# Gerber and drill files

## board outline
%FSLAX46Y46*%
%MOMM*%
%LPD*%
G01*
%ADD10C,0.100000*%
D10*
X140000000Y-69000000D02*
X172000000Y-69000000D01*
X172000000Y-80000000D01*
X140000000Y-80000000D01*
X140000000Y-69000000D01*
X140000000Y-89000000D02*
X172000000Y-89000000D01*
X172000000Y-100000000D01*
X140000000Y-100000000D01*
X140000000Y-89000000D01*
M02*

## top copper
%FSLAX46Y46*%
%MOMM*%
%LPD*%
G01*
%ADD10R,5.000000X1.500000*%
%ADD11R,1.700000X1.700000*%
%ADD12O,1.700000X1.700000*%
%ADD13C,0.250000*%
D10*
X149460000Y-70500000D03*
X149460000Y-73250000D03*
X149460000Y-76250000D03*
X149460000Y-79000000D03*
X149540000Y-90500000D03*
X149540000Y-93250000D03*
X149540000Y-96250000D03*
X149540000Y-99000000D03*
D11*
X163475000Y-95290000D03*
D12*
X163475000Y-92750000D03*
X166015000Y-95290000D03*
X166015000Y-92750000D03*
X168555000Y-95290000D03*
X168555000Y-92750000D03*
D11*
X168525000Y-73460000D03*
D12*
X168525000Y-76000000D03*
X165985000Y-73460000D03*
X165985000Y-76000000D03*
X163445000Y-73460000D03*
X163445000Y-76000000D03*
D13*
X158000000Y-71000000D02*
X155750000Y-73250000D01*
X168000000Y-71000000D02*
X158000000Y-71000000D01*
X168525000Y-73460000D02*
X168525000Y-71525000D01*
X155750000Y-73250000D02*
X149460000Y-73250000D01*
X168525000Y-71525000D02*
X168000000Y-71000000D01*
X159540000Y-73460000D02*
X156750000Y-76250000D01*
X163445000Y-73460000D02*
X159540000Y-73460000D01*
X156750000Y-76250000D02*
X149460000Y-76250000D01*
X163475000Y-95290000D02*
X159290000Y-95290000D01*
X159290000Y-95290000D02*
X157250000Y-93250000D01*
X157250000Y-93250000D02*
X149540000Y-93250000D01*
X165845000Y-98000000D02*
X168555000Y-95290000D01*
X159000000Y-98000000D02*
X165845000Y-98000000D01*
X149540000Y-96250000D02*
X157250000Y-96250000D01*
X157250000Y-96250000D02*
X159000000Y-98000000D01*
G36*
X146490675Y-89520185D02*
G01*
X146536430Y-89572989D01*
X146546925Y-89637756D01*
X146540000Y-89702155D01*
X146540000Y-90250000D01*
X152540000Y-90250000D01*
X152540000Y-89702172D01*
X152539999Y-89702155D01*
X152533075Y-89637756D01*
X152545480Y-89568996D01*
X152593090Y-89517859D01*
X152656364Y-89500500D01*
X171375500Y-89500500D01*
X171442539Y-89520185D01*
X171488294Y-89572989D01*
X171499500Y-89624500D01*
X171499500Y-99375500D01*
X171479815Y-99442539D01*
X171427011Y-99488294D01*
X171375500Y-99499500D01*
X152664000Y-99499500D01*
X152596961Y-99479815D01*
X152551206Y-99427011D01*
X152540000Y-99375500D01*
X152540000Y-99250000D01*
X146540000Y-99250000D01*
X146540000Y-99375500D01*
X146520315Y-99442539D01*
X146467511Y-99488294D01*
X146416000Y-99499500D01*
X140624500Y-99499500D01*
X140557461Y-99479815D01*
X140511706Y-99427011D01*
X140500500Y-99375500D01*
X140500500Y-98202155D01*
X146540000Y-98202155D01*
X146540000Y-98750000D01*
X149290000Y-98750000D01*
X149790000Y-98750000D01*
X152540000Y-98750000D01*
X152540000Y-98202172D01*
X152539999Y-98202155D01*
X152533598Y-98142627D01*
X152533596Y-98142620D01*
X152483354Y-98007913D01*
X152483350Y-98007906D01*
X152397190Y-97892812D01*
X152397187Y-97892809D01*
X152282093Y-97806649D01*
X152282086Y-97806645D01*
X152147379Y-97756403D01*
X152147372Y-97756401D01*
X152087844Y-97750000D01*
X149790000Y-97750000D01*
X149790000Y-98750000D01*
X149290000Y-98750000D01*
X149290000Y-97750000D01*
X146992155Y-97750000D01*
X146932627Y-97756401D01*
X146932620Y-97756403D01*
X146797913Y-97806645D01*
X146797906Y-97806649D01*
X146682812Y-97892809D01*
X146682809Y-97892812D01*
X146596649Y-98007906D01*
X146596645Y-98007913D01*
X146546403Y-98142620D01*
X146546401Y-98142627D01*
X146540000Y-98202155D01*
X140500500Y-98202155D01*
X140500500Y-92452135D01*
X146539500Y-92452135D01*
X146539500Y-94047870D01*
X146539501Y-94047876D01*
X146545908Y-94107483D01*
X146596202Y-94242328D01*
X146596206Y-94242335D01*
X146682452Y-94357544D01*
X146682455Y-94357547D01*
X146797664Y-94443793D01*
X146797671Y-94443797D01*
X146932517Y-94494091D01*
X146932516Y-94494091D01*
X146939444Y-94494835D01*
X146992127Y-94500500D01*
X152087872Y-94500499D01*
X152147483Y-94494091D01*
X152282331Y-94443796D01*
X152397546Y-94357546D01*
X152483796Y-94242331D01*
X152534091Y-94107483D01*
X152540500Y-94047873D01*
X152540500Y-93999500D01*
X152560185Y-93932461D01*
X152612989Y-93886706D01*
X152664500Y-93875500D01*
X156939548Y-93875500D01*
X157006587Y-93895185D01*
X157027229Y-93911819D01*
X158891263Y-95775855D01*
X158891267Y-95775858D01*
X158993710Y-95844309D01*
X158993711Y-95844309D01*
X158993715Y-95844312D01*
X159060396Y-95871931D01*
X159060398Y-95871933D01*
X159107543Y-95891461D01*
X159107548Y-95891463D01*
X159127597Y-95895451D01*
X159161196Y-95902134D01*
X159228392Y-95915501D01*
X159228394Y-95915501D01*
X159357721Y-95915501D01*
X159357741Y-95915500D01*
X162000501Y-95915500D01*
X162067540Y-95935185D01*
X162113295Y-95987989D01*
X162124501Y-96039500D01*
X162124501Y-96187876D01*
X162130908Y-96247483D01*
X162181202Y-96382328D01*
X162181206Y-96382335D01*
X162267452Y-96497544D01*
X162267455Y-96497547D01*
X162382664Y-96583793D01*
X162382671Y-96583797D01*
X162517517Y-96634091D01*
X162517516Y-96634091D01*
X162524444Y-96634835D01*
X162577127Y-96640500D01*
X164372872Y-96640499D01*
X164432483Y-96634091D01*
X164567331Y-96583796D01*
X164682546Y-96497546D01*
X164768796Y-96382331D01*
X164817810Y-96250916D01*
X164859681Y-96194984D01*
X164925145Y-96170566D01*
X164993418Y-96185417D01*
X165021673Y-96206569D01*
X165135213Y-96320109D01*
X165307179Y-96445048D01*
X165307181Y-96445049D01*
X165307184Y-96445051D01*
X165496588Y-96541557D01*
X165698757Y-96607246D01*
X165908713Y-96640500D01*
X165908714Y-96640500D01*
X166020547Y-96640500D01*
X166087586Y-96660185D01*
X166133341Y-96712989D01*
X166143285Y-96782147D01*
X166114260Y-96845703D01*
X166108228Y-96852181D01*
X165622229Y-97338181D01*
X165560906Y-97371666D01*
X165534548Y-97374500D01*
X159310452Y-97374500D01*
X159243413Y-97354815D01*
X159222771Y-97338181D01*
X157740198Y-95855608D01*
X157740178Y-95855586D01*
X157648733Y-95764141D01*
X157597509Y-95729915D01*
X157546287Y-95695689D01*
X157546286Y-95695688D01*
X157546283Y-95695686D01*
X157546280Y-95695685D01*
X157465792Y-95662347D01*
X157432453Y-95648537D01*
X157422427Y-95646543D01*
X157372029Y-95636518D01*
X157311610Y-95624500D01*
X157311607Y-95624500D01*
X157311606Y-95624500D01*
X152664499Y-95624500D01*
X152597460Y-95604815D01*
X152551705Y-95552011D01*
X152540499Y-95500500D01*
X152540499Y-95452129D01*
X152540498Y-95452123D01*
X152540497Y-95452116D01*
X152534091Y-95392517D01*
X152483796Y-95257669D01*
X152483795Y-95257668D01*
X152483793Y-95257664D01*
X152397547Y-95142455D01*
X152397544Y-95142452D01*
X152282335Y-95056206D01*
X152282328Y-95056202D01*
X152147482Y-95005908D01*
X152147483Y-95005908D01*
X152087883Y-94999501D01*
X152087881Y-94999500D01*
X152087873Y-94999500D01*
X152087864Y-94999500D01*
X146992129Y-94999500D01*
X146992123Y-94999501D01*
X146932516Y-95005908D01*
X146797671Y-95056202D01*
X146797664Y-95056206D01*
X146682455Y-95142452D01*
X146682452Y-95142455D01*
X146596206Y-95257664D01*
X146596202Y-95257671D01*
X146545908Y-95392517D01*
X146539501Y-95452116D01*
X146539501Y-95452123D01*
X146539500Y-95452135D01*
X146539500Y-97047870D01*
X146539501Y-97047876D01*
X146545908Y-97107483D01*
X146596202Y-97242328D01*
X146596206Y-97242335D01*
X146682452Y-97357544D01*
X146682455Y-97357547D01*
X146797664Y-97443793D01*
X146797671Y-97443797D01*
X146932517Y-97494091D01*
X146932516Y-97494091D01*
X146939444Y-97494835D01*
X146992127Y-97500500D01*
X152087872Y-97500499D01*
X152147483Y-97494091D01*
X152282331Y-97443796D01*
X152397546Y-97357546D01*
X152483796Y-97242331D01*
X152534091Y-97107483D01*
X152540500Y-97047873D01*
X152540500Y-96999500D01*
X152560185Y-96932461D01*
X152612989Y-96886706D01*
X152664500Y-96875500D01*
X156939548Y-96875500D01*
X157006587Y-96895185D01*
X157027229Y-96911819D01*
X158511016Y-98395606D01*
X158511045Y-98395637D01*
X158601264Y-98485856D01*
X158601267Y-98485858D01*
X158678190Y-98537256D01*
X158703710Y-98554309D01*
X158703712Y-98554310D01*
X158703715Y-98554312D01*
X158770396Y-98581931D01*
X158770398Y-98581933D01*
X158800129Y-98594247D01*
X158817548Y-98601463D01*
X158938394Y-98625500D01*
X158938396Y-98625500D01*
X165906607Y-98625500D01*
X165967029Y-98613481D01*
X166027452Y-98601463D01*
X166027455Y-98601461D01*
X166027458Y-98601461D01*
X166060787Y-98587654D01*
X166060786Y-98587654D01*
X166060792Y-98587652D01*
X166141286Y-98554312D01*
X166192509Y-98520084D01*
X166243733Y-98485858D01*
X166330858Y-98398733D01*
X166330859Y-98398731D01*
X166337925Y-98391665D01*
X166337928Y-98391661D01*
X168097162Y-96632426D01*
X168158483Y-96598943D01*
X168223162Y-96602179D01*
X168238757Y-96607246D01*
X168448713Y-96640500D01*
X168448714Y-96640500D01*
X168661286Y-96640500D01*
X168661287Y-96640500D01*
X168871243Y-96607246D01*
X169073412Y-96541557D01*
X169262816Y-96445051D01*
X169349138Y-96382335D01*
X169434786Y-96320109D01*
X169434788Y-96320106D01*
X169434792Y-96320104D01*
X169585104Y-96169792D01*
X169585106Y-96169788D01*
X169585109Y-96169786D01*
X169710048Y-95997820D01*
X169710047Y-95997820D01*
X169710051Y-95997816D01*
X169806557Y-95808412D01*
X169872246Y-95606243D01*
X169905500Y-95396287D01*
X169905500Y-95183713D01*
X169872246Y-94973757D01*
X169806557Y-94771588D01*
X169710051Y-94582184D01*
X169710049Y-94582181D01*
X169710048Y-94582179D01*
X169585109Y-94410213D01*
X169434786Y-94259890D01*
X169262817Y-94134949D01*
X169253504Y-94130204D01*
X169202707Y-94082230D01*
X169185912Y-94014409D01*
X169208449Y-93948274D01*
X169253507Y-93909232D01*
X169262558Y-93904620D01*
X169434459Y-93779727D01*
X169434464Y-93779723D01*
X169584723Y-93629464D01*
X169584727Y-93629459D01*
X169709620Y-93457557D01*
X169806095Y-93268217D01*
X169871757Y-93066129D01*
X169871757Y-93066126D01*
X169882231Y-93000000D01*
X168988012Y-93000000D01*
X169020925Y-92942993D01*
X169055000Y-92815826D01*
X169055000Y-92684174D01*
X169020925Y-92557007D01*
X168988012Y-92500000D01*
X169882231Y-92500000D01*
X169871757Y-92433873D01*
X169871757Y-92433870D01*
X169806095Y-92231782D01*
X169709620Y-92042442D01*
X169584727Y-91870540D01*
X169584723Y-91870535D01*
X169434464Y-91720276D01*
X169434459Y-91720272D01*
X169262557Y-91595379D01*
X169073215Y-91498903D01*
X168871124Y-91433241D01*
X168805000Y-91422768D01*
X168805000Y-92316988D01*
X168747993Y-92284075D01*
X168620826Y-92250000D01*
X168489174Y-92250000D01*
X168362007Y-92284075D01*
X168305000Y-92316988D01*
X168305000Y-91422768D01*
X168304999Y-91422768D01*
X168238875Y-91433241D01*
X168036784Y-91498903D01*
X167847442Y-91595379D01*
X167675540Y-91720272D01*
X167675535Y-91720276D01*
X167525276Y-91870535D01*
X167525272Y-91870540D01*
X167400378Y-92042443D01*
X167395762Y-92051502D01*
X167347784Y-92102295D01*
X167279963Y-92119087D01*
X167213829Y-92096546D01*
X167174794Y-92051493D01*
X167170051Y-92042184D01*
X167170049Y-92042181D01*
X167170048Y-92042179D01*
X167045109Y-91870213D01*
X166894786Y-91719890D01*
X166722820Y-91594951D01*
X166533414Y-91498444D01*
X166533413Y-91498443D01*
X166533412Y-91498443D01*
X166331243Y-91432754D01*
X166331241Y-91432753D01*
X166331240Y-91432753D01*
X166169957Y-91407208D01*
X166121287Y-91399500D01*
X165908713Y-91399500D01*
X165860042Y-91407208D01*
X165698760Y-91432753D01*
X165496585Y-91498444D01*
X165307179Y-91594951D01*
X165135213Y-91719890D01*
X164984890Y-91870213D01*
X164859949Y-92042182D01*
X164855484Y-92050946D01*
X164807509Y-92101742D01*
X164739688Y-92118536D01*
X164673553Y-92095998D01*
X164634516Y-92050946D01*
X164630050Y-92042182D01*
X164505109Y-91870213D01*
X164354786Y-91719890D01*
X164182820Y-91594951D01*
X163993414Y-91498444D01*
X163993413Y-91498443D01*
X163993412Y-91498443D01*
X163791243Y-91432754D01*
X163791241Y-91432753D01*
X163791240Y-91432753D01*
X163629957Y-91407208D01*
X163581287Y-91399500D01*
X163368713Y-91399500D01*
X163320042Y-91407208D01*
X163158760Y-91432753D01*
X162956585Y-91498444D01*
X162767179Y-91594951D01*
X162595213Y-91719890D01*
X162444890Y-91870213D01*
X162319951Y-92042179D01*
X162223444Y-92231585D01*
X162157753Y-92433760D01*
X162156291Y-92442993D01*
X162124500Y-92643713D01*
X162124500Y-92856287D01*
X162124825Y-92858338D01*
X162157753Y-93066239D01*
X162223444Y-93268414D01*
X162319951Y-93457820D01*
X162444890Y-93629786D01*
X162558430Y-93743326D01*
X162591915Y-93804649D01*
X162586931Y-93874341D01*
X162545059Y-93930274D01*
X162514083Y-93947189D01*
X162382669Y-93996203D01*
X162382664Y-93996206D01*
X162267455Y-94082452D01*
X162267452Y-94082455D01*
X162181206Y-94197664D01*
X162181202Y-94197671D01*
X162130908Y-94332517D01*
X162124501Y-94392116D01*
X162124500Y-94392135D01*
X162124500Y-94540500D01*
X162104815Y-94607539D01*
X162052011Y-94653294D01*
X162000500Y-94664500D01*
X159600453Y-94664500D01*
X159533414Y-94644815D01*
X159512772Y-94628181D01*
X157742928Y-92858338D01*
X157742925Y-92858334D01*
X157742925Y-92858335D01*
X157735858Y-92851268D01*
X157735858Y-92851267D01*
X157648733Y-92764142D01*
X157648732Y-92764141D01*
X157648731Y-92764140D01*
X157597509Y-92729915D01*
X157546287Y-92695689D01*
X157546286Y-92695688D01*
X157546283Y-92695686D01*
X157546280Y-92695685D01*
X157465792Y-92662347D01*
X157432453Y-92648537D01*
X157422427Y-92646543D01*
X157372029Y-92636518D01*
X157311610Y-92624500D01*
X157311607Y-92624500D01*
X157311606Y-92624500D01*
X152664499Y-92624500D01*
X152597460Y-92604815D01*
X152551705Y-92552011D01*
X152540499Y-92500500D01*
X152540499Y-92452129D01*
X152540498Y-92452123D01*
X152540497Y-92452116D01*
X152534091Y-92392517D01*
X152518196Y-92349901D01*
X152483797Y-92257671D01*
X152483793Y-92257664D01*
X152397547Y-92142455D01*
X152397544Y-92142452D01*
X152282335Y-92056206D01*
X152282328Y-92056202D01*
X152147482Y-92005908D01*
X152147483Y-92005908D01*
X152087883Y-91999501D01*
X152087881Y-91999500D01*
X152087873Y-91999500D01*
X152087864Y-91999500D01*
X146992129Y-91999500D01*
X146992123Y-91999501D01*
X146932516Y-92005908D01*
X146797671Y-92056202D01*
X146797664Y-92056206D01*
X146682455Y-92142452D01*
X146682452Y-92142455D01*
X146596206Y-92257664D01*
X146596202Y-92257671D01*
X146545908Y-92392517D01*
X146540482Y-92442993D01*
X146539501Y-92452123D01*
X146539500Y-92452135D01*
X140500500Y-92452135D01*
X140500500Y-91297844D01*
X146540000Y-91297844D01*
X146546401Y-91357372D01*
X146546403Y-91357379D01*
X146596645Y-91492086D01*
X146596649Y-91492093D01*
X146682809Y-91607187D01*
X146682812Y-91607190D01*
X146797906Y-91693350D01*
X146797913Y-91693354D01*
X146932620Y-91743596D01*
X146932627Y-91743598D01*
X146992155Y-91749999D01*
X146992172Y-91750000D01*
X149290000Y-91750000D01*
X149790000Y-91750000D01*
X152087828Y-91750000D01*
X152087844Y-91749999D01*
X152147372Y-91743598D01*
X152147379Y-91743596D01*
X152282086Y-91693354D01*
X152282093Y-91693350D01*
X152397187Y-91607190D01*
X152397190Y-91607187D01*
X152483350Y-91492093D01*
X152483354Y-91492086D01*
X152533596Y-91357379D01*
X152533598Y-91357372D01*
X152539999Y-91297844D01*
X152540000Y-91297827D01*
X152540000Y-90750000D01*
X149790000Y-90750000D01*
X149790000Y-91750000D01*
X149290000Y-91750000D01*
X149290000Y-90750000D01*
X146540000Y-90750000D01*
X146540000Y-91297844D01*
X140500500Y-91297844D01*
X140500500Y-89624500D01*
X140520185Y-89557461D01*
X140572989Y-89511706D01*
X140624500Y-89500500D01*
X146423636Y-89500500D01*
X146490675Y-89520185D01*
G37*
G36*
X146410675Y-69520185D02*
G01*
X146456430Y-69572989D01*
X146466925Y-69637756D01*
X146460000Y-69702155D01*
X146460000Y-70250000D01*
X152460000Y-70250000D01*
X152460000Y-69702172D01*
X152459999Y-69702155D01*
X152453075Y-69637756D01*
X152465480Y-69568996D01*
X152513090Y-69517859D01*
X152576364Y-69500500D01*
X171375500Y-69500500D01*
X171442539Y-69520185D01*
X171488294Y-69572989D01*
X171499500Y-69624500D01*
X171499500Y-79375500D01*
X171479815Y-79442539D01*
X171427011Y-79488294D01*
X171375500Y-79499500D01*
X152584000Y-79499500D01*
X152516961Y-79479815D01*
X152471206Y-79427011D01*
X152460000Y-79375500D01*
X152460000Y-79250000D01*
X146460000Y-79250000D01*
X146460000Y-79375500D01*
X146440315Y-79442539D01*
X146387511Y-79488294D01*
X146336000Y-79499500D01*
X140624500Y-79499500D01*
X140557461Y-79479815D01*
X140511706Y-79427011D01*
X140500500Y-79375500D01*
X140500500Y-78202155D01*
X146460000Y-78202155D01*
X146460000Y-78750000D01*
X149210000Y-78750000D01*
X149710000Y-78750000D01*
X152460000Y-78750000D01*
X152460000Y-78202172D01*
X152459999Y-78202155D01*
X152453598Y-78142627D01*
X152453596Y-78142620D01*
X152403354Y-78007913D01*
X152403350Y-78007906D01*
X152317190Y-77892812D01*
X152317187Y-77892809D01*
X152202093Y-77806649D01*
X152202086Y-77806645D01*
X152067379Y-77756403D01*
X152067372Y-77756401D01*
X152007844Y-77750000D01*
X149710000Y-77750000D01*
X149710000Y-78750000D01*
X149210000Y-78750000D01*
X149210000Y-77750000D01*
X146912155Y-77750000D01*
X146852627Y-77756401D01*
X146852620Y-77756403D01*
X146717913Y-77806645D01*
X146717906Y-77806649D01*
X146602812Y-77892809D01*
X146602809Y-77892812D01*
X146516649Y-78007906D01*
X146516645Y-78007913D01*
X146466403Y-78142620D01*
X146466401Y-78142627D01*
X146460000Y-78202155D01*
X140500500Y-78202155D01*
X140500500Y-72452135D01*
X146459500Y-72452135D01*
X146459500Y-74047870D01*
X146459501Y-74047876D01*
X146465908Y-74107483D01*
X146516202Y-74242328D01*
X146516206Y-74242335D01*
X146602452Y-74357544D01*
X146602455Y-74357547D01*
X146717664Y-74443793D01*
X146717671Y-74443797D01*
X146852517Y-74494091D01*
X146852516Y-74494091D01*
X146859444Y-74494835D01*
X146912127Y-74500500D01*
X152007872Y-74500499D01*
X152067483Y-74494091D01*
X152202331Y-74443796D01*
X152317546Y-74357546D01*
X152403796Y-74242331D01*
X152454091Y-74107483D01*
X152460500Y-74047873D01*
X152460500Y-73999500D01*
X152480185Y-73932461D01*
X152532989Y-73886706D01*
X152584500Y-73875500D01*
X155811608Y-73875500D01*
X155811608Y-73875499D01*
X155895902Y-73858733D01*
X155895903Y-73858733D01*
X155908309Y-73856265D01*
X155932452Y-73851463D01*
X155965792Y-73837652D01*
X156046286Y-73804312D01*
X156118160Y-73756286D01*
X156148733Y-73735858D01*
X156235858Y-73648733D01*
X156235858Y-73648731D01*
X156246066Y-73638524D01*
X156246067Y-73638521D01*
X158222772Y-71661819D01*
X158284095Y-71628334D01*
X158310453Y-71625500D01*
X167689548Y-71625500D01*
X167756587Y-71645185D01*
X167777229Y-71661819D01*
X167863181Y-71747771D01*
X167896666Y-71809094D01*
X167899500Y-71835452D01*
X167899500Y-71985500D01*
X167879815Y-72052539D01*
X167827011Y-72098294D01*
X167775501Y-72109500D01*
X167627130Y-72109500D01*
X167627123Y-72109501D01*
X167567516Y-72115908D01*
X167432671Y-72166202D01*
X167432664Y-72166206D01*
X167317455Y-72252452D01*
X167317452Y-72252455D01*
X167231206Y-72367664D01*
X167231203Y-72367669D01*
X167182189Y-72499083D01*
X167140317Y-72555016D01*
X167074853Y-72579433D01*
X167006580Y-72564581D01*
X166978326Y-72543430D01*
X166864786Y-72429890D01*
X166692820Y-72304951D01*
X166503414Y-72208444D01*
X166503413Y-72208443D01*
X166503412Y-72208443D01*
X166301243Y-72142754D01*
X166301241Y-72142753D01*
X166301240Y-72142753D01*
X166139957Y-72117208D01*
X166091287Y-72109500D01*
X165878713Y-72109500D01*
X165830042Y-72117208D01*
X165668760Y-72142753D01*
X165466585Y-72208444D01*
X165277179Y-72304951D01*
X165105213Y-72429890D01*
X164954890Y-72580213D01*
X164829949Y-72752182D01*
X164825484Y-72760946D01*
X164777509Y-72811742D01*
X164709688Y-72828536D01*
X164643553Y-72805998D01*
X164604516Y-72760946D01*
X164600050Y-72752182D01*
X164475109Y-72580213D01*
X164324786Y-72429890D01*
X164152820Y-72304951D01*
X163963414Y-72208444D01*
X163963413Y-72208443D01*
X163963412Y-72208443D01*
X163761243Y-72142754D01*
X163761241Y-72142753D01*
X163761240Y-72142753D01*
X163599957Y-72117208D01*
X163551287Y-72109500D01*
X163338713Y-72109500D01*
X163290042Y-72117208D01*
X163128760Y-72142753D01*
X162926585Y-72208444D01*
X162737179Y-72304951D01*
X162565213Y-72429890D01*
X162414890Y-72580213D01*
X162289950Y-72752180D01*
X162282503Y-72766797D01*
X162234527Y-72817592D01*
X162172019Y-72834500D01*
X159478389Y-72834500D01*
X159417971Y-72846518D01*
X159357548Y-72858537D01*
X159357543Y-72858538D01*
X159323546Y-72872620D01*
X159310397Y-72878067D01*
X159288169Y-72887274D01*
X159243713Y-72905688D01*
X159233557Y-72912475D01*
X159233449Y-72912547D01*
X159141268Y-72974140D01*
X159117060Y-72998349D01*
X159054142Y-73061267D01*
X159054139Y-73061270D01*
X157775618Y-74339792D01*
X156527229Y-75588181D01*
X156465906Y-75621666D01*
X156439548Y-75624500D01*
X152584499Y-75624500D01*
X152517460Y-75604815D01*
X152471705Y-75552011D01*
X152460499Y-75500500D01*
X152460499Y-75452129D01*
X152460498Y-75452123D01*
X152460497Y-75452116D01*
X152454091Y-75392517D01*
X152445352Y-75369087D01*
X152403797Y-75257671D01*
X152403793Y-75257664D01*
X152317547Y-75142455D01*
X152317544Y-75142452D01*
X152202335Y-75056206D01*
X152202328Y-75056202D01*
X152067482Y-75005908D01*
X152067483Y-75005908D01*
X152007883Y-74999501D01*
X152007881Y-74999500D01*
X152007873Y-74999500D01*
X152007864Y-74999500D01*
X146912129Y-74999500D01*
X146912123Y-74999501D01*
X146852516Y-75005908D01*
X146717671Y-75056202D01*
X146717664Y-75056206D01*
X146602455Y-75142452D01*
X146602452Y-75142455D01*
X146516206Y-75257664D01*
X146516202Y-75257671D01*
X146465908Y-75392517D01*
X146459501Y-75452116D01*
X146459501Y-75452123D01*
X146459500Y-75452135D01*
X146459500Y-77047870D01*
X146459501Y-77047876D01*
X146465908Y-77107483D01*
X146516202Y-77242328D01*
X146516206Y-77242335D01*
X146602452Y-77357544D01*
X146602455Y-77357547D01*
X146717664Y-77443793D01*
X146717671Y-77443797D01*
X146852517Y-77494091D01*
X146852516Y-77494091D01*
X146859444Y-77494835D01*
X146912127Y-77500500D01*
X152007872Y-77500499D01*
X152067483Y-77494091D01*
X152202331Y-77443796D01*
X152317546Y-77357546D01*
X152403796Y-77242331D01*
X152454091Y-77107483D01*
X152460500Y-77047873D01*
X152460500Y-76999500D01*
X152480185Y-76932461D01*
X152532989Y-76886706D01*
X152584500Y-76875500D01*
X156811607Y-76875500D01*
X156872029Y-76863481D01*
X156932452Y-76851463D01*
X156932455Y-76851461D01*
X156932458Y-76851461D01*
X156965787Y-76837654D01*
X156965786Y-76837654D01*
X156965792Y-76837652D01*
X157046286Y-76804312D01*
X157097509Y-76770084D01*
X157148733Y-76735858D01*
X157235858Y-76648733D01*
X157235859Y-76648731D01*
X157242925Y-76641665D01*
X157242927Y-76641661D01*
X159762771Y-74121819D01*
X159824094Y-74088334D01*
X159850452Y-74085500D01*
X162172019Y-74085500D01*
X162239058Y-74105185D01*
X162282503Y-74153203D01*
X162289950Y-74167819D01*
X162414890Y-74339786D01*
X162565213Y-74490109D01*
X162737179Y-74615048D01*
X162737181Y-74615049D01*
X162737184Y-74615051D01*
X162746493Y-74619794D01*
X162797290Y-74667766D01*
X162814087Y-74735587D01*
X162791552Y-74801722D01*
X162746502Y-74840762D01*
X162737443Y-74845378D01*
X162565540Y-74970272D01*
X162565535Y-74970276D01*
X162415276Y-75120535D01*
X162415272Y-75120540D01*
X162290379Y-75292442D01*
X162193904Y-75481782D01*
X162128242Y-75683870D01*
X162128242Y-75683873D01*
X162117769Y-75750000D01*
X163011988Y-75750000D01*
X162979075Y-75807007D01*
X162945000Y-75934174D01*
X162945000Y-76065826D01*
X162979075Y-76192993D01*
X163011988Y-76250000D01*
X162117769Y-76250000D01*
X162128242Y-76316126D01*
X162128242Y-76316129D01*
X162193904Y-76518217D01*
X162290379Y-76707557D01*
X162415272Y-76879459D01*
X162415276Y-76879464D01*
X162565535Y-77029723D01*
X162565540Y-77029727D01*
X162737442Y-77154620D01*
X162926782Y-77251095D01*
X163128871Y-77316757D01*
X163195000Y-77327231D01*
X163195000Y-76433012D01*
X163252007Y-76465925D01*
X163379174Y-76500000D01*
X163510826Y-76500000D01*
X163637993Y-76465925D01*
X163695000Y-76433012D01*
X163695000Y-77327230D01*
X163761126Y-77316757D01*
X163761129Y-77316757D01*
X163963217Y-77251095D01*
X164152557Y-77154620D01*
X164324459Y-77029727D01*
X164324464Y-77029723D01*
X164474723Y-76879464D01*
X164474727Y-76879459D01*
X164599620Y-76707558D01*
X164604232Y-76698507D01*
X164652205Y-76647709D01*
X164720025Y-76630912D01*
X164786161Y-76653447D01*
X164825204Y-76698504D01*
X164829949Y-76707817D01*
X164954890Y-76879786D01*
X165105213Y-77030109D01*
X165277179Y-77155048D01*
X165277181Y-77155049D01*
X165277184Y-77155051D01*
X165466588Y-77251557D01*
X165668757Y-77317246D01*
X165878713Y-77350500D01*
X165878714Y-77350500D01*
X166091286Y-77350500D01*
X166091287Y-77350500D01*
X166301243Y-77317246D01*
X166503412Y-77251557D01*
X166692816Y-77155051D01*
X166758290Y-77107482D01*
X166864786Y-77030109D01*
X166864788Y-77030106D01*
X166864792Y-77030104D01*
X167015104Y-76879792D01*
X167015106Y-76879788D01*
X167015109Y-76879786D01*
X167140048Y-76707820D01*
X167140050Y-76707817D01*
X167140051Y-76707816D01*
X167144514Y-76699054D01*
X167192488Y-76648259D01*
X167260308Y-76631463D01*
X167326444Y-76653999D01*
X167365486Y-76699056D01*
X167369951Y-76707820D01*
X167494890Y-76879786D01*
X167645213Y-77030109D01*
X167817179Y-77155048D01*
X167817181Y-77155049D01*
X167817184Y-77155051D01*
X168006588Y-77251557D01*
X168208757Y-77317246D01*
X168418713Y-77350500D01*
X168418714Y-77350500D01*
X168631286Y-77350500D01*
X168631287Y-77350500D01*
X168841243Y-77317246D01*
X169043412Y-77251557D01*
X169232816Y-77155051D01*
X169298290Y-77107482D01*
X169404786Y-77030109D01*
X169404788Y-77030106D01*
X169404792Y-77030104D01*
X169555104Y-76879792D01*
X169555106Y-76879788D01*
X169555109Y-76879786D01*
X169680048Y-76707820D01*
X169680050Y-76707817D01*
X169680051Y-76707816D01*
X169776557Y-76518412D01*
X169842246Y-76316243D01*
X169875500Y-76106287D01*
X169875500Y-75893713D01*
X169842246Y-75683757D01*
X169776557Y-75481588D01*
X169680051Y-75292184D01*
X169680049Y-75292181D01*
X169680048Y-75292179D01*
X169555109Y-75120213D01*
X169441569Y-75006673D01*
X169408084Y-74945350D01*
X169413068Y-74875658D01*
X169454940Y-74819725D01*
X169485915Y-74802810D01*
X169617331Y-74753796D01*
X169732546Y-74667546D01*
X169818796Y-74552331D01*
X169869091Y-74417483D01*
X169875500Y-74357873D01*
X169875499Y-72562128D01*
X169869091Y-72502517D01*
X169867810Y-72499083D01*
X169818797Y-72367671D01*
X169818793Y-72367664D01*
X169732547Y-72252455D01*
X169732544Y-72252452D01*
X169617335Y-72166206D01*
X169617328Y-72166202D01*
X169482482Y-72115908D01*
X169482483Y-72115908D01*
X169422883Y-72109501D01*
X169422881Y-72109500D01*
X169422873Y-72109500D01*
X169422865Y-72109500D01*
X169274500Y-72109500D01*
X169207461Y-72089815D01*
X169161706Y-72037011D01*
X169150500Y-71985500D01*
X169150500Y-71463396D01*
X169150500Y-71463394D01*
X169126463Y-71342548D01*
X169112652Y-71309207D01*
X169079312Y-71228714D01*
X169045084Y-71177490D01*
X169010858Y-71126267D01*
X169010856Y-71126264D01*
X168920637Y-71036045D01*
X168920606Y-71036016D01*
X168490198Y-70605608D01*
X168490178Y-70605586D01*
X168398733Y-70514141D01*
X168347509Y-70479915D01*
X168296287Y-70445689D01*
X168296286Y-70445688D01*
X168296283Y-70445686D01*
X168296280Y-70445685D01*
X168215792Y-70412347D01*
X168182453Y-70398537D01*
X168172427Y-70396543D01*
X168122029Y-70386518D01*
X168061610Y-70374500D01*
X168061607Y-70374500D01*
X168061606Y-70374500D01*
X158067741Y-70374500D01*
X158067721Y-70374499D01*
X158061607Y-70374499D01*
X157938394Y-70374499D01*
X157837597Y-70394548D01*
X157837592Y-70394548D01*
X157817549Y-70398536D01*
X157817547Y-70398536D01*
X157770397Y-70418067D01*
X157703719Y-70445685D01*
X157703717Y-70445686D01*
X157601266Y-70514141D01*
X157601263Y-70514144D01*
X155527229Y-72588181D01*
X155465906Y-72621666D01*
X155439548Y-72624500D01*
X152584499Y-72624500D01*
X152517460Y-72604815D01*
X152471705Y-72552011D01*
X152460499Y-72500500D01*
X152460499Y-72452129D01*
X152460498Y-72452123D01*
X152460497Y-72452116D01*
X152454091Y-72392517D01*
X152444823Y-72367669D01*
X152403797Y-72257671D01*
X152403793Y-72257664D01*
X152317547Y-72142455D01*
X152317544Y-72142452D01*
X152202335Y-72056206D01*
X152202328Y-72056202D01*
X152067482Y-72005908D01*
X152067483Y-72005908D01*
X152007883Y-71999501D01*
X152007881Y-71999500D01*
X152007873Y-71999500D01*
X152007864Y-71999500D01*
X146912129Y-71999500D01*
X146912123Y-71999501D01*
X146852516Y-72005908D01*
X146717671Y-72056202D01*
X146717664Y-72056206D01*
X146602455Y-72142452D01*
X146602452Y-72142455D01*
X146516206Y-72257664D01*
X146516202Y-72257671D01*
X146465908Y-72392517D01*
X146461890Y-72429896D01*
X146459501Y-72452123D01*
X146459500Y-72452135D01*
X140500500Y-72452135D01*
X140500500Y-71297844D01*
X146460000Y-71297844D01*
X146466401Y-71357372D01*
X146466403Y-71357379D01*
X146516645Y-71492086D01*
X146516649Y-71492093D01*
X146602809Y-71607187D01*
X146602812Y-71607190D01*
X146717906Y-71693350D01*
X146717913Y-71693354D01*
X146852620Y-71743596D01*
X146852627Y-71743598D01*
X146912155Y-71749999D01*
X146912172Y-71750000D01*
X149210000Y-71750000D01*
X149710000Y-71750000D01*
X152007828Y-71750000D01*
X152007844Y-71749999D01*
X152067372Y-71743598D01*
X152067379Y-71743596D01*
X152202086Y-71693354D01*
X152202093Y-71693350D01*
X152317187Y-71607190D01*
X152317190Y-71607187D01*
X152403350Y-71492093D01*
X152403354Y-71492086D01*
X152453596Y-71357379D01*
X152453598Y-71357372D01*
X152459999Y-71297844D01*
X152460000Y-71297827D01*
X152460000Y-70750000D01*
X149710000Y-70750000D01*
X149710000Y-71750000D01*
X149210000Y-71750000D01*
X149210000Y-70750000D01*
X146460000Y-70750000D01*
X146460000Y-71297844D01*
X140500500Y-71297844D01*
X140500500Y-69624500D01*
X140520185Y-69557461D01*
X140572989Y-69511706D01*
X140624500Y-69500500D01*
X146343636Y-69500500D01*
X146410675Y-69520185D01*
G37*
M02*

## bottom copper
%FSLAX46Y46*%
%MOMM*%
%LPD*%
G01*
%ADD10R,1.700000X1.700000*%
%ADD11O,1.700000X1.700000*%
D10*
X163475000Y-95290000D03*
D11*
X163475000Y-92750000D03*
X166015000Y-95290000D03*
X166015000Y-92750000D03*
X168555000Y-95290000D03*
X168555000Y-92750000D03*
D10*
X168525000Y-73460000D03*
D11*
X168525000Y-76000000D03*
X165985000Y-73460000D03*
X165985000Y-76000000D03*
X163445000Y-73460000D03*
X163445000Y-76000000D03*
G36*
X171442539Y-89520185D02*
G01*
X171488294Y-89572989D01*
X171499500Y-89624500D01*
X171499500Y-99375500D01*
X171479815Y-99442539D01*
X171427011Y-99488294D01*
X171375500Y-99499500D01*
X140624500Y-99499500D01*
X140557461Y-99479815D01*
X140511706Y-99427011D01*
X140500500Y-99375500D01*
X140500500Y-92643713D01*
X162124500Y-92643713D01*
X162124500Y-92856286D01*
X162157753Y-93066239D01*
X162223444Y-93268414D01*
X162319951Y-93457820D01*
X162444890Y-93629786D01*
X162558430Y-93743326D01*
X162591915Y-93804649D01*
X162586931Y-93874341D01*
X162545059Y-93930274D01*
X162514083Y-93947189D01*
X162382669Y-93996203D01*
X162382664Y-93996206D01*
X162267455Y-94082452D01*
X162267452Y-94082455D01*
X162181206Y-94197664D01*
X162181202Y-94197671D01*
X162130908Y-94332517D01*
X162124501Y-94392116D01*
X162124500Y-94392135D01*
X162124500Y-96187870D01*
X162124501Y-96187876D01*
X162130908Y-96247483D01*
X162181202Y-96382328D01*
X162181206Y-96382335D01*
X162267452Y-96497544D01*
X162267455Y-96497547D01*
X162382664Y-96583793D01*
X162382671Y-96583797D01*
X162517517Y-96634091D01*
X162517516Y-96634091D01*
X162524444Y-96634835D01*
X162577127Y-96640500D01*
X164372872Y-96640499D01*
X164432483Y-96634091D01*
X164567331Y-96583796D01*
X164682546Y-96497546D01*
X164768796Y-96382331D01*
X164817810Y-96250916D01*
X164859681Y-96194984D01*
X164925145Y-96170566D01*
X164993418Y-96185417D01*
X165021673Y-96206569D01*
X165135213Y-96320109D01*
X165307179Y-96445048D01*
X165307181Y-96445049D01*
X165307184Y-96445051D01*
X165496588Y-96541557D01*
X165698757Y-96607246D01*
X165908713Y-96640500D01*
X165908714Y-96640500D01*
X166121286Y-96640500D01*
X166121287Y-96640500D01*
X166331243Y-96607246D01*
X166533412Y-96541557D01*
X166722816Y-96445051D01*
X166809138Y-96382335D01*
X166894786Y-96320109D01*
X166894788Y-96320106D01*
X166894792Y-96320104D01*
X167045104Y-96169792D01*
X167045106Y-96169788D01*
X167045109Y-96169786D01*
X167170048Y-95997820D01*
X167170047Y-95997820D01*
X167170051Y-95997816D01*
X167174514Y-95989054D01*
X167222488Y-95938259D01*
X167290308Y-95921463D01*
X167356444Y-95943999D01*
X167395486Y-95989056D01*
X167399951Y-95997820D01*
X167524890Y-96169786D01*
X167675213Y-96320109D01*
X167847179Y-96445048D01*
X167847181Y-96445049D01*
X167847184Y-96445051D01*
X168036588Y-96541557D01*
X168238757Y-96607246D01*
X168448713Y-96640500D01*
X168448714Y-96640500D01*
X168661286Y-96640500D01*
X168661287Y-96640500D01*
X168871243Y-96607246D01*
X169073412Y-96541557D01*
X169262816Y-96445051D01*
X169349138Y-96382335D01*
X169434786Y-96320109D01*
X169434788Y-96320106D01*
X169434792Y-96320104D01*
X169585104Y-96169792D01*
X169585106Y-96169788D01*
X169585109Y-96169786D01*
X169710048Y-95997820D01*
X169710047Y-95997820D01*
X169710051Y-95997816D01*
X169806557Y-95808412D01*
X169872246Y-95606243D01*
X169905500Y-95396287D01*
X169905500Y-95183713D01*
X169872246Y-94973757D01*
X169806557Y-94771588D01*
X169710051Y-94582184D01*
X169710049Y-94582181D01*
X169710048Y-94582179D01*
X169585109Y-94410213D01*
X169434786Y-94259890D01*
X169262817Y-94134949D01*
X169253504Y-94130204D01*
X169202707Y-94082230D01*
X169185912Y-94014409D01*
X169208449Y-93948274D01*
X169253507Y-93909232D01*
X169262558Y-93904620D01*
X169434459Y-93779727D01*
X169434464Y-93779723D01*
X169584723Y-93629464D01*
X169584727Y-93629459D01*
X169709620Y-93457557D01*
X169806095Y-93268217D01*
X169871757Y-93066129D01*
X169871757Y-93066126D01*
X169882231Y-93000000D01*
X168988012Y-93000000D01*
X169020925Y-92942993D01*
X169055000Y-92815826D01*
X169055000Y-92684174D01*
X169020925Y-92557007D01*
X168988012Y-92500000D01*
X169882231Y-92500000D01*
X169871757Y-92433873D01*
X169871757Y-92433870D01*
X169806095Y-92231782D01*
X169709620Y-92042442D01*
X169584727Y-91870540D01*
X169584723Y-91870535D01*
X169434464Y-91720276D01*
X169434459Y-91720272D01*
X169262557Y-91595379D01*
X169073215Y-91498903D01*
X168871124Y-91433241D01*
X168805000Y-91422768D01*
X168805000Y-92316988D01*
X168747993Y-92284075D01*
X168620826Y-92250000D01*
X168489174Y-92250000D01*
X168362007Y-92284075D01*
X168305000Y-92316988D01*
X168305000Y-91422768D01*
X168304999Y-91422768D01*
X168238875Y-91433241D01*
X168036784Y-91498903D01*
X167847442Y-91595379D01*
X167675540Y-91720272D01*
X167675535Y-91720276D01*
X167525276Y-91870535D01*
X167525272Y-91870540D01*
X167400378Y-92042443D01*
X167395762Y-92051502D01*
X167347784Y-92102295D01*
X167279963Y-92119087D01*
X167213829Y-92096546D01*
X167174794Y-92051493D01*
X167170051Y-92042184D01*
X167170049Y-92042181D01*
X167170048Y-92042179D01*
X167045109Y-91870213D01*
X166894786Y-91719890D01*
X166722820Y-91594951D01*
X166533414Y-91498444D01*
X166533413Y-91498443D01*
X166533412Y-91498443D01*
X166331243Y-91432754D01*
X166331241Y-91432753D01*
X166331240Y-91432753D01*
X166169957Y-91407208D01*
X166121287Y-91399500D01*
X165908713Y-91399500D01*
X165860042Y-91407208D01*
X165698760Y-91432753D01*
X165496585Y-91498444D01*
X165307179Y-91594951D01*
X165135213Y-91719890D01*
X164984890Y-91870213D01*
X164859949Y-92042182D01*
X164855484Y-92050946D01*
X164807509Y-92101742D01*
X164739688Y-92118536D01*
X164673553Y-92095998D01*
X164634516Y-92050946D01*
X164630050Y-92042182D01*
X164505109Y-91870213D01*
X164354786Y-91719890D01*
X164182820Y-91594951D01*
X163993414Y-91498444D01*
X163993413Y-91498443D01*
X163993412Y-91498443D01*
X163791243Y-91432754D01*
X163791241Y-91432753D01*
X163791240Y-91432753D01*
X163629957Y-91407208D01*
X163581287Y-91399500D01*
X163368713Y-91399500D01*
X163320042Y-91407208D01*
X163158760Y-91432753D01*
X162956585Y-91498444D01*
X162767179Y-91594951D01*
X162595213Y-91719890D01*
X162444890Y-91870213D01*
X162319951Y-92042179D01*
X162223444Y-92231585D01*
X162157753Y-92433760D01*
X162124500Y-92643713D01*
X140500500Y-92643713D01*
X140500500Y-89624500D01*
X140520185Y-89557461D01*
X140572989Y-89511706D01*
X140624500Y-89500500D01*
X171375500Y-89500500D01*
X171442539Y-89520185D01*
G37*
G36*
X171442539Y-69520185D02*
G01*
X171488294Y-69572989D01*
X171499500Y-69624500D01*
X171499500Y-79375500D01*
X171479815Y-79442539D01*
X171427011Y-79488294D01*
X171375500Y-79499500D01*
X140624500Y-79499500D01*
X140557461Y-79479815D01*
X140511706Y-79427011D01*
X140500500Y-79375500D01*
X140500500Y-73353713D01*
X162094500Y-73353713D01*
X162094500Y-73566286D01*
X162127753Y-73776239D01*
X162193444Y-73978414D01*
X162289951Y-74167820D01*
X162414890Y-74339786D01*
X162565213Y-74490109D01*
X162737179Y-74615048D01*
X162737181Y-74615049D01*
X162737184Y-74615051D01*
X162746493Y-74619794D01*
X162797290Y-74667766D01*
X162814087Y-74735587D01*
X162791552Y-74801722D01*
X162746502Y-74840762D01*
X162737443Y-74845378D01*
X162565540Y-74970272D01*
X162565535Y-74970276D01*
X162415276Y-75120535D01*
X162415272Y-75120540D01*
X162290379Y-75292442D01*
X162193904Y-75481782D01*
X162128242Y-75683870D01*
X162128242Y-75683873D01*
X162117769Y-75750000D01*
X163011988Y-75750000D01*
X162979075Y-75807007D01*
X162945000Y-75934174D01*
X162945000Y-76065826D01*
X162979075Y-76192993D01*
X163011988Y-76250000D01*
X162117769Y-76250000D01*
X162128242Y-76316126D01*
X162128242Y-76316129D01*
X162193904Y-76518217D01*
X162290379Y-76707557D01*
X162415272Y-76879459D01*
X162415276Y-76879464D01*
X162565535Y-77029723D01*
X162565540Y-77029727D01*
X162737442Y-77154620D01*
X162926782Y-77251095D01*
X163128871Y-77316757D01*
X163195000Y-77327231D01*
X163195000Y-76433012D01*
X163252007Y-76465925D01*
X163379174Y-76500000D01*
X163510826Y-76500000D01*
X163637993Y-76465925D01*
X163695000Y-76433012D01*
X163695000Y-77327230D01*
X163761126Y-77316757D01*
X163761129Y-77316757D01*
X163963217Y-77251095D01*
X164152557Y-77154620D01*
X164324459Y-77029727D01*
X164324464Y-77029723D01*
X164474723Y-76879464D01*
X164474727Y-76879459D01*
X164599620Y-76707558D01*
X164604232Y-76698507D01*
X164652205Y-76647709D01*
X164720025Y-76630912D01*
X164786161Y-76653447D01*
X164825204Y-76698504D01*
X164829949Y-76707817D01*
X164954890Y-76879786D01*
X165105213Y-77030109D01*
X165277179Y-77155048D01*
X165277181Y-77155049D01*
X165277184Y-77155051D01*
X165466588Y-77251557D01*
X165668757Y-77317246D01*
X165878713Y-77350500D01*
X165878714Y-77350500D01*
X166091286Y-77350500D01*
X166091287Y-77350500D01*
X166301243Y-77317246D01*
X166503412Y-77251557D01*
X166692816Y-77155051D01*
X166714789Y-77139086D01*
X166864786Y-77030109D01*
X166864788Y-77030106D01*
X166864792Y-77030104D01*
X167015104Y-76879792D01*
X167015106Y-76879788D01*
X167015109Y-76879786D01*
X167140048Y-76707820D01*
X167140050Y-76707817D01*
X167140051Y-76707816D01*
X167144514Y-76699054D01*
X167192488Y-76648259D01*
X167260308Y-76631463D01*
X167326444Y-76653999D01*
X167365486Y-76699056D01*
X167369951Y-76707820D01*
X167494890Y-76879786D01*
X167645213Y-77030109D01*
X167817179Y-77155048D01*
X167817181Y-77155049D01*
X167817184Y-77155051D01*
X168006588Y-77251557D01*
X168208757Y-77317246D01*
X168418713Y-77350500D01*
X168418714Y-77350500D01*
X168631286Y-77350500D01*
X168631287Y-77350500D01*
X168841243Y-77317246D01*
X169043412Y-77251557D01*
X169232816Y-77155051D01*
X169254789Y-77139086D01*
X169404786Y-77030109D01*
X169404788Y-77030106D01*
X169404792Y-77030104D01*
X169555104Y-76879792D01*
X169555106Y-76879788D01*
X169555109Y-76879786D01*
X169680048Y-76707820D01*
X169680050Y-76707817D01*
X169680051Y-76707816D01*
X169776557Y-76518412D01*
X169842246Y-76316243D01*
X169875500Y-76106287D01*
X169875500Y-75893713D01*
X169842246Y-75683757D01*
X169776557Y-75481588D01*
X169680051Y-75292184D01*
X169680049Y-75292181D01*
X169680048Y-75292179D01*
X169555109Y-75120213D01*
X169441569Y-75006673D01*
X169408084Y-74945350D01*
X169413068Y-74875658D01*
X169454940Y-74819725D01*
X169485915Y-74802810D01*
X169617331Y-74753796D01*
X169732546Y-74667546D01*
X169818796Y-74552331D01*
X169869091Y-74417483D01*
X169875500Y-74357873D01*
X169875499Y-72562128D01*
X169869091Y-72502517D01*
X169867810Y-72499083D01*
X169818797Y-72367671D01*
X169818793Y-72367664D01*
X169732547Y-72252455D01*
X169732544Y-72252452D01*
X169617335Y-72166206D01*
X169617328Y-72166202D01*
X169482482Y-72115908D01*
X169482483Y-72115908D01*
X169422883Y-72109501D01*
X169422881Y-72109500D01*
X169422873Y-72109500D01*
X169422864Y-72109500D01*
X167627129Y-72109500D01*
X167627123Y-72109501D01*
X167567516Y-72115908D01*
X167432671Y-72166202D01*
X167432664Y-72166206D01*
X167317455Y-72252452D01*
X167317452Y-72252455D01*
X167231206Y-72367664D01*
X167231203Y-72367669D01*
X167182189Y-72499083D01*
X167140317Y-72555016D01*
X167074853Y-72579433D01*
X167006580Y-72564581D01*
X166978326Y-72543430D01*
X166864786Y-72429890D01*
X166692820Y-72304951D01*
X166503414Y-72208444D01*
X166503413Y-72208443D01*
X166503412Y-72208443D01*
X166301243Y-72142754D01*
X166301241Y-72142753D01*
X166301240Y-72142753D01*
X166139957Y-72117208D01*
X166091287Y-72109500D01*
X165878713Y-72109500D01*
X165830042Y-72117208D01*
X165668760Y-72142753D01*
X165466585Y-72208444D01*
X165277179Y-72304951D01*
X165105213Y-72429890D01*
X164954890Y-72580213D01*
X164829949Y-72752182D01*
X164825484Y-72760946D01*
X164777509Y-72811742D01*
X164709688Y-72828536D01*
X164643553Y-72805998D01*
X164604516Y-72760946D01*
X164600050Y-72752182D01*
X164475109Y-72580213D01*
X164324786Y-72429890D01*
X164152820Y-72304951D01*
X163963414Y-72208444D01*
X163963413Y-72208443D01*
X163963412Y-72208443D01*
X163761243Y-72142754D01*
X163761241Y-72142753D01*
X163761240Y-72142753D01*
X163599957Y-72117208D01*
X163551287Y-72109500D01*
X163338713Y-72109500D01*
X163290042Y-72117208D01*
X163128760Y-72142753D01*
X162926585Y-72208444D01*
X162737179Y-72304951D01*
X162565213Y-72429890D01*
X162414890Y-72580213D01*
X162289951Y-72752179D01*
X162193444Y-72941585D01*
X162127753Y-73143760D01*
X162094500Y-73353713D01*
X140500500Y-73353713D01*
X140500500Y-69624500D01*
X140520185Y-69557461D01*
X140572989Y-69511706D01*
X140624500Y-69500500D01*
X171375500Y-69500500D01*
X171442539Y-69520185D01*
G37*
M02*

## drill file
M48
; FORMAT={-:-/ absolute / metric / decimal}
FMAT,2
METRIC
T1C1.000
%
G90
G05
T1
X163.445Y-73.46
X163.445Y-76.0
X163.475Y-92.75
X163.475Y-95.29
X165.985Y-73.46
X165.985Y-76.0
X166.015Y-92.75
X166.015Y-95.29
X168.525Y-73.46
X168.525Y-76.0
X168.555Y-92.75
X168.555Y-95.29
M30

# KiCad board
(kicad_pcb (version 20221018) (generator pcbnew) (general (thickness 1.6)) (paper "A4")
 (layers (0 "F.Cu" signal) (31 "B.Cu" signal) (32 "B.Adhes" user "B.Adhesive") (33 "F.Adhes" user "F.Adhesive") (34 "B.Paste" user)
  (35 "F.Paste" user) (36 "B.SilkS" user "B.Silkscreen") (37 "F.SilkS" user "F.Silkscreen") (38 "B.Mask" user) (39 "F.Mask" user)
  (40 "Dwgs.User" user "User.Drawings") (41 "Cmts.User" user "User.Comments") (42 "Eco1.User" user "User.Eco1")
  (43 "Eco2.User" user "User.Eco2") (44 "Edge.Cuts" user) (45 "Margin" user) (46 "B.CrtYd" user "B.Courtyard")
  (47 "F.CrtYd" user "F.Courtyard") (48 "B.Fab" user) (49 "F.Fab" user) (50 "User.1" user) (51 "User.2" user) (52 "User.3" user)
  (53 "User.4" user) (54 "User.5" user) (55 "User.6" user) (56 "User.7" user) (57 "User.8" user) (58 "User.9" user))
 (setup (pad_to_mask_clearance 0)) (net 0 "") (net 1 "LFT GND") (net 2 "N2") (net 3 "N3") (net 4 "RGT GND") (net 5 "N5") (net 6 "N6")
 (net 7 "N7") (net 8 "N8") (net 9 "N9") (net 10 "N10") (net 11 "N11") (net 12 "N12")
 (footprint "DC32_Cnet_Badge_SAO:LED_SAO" (layer "F.Cu") (at 118.46 74.75)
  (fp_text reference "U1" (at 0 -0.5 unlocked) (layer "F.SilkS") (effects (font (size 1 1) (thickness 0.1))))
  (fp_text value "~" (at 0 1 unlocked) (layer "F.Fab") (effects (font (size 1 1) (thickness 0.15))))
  (pad "1" smd rect (at 31 -4.25) (size 5 1.5) (layers "F.Cu" "F.Paste" "F.Mask") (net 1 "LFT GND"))
  (pad "2" smd rect (at 31 -1.5) (size 5 1.5) (layers "F.Cu" "F.Paste" "F.Mask") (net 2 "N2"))
  (pad "3" smd rect (at 31 1.5) (size 5 1.5) (layers "F.Cu" "F.Paste" "F.Mask") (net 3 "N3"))
  (pad "4" smd rect (at 31 4.25) (size 5 1.5) (layers "F.Cu" "F.Paste" "F.Mask") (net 1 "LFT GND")))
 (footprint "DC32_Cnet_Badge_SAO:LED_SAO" (layer "F.Cu") (at 118.54 94.75)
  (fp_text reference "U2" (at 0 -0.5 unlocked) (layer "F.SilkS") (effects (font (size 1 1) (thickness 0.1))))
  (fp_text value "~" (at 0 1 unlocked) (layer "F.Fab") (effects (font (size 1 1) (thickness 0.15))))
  (pad "1" smd rect (at 31 -4.25) (size 5 1.5) (layers "F.Cu" "F.Paste" "F.Mask") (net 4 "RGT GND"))
  (pad "2" smd rect (at 31 -1.5) (size 5 1.5) (layers "F.Cu" "F.Paste" "F.Mask") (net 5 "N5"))
  (pad "3" smd rect (at 31 1.5) (size 5 1.5) (layers "F.Cu" "F.Paste" "F.Mask") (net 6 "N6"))
  (pad "4" smd rect (at 31 4.25) (size 5 1.5) (layers "F.Cu" "F.Paste" "F.Mask") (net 4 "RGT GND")))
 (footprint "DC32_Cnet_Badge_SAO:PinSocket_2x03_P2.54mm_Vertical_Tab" (layer "B.Cu") (at 163.475 95.29 -90)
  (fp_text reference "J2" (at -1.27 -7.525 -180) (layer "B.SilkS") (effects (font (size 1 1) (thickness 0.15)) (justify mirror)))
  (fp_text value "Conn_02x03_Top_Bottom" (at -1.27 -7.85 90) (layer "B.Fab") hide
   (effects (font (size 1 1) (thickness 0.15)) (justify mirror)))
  (pad "1" thru_hole rect (at 0 0 270) (size 1.7 1.7) (drill 1) (layers "*.Cu" "*.Mask") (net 5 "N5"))
  (pad "2" thru_hole oval (at -2.54 0 270) (size 1.7 1.7) (drill 1) (layers "*.Cu" "*.Mask") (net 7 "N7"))
  (pad "3" thru_hole oval (at 0 -2.54 270) (size 1.7 1.7) (drill 1) (layers "*.Cu" "*.Mask") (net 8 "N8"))
  (pad "4" thru_hole oval (at -2.54 -2.54 270) (size 1.7 1.7) (drill 1) (layers "*.Cu" "*.Mask") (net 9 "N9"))
  (pad "5" thru_hole oval (at 0 -5.08 270) (size 1.7 1.7) (drill 1) (layers "*.Cu" "*.Mask") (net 6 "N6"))
  (pad "6" thru_hole oval (at -2.54 -5.08 270) (size 1.7 1.7) (drill 1) (layers "*.Cu" "*.Mask") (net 4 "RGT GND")))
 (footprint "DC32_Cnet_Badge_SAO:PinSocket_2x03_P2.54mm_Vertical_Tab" (layer "B.Cu") (at 168.525 73.46 90)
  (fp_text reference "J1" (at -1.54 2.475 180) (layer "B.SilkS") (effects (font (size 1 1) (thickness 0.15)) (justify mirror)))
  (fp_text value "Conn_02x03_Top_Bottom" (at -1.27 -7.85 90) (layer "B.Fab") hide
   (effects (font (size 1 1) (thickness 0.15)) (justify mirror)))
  (pad "1" thru_hole rect (at 0 0 90) (size 1.7 1.7) (drill 1) (layers "*.Cu" "*.Mask") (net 2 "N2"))
  (pad "2" thru_hole oval (at -2.54 0 90) (size 1.7 1.7) (drill 1) (layers "*.Cu" "*.Mask") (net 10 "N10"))
  (pad "3" thru_hole oval (at 0 -2.54 90) (size 1.7 1.7) (drill 1) (layers "*.Cu" "*.Mask") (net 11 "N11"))
  (pad "4" thru_hole oval (at -2.54 -2.54 90) (size 1.7 1.7) (drill 1) (layers "*.Cu" "*.Mask") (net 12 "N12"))
  (pad "5" thru_hole oval (at 0 -5.08 90) (size 1.7 1.7) (drill 1) (layers "*.Cu" "*.Mask") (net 3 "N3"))
  (pad "6" thru_hole oval (at -2.54 -5.08 90) (size 1.7 1.7) (drill 1) (layers "*.Cu" "*.Mask") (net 1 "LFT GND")))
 (gr_rect (start 140 69) (end 172 80) (stroke (width 0.1) (type default)) (fill none) (layer "Edge.Cuts"))
 (gr_rect (start 140 89) (end 172 100) (stroke (width 0.1) (type default)) (fill none) (layer "Edge.Cuts"))
 (segment (start 158 71) (end 155.75 73.25) (width 0.25) (layer "F.Cu") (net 2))
 (segment (start 168 71) (end 158 71) (width 0.25) (layer "F.Cu") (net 2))
 (segment (start 168.525 73.46) (end 168.525 71.525) (width 0.25) (layer "F.Cu") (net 2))
 (segment (start 155.75 73.25) (end 149.46 73.25) (width 0.25) (layer "F.Cu") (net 2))
 (segment (start 168.525 71.525) (end 168 71) (width 0.25) (layer "F.Cu") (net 2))
 (segment (start 159.54 73.46) (end 156.75 76.25) (width 0.25) (layer "F.Cu") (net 3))
 (segment (start 163.445 73.46) (end 159.54 73.46) (width 0.25) (layer "F.Cu") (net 3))
 (segment (start 156.75 76.25) (end 149.46 76.25) (width 0.25) (layer "F.Cu") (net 3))
 (segment (start 163.475 95.29) (end 159.29 95.29) (width 0.25) (layer "F.Cu") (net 5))
 (segment (start 159.29 95.29) (end 157.25 93.25) (width 0.25) (layer "F.Cu") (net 5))
 (segment (start 157.25 93.25) (end 149.54 93.25) (width 0.25) (layer "F.Cu") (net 5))
 (segment (start 165.845 98) (end 168.555 95.29) (width 0.25) (layer "F.Cu") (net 6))
 (segment (start 159 98) (end 165.845 98) (width 0.25) (layer "F.Cu") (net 6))
 (segment (start 149.54 96.25) (end 157.25 96.25) (width 0.25) (layer "F.Cu") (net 6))
 (segment (start 157.25 96.25) (end 159 98) (width 0.25) (layer "F.Cu") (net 6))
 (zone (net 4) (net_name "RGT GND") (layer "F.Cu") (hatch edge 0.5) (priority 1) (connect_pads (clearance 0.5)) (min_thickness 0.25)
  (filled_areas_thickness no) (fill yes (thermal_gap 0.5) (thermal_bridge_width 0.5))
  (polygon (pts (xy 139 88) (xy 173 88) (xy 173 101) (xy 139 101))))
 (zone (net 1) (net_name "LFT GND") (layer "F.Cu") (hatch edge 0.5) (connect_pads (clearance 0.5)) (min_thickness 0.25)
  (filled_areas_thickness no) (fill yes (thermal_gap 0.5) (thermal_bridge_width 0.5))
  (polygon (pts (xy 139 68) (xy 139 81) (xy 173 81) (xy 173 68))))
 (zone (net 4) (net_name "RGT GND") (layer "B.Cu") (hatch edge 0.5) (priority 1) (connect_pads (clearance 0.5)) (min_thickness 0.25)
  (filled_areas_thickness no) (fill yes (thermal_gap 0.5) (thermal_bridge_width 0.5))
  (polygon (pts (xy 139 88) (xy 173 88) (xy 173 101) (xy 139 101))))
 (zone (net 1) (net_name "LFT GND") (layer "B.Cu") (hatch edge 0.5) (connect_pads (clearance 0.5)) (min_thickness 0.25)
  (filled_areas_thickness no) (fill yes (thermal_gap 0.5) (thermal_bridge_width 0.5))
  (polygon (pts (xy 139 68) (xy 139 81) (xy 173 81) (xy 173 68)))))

